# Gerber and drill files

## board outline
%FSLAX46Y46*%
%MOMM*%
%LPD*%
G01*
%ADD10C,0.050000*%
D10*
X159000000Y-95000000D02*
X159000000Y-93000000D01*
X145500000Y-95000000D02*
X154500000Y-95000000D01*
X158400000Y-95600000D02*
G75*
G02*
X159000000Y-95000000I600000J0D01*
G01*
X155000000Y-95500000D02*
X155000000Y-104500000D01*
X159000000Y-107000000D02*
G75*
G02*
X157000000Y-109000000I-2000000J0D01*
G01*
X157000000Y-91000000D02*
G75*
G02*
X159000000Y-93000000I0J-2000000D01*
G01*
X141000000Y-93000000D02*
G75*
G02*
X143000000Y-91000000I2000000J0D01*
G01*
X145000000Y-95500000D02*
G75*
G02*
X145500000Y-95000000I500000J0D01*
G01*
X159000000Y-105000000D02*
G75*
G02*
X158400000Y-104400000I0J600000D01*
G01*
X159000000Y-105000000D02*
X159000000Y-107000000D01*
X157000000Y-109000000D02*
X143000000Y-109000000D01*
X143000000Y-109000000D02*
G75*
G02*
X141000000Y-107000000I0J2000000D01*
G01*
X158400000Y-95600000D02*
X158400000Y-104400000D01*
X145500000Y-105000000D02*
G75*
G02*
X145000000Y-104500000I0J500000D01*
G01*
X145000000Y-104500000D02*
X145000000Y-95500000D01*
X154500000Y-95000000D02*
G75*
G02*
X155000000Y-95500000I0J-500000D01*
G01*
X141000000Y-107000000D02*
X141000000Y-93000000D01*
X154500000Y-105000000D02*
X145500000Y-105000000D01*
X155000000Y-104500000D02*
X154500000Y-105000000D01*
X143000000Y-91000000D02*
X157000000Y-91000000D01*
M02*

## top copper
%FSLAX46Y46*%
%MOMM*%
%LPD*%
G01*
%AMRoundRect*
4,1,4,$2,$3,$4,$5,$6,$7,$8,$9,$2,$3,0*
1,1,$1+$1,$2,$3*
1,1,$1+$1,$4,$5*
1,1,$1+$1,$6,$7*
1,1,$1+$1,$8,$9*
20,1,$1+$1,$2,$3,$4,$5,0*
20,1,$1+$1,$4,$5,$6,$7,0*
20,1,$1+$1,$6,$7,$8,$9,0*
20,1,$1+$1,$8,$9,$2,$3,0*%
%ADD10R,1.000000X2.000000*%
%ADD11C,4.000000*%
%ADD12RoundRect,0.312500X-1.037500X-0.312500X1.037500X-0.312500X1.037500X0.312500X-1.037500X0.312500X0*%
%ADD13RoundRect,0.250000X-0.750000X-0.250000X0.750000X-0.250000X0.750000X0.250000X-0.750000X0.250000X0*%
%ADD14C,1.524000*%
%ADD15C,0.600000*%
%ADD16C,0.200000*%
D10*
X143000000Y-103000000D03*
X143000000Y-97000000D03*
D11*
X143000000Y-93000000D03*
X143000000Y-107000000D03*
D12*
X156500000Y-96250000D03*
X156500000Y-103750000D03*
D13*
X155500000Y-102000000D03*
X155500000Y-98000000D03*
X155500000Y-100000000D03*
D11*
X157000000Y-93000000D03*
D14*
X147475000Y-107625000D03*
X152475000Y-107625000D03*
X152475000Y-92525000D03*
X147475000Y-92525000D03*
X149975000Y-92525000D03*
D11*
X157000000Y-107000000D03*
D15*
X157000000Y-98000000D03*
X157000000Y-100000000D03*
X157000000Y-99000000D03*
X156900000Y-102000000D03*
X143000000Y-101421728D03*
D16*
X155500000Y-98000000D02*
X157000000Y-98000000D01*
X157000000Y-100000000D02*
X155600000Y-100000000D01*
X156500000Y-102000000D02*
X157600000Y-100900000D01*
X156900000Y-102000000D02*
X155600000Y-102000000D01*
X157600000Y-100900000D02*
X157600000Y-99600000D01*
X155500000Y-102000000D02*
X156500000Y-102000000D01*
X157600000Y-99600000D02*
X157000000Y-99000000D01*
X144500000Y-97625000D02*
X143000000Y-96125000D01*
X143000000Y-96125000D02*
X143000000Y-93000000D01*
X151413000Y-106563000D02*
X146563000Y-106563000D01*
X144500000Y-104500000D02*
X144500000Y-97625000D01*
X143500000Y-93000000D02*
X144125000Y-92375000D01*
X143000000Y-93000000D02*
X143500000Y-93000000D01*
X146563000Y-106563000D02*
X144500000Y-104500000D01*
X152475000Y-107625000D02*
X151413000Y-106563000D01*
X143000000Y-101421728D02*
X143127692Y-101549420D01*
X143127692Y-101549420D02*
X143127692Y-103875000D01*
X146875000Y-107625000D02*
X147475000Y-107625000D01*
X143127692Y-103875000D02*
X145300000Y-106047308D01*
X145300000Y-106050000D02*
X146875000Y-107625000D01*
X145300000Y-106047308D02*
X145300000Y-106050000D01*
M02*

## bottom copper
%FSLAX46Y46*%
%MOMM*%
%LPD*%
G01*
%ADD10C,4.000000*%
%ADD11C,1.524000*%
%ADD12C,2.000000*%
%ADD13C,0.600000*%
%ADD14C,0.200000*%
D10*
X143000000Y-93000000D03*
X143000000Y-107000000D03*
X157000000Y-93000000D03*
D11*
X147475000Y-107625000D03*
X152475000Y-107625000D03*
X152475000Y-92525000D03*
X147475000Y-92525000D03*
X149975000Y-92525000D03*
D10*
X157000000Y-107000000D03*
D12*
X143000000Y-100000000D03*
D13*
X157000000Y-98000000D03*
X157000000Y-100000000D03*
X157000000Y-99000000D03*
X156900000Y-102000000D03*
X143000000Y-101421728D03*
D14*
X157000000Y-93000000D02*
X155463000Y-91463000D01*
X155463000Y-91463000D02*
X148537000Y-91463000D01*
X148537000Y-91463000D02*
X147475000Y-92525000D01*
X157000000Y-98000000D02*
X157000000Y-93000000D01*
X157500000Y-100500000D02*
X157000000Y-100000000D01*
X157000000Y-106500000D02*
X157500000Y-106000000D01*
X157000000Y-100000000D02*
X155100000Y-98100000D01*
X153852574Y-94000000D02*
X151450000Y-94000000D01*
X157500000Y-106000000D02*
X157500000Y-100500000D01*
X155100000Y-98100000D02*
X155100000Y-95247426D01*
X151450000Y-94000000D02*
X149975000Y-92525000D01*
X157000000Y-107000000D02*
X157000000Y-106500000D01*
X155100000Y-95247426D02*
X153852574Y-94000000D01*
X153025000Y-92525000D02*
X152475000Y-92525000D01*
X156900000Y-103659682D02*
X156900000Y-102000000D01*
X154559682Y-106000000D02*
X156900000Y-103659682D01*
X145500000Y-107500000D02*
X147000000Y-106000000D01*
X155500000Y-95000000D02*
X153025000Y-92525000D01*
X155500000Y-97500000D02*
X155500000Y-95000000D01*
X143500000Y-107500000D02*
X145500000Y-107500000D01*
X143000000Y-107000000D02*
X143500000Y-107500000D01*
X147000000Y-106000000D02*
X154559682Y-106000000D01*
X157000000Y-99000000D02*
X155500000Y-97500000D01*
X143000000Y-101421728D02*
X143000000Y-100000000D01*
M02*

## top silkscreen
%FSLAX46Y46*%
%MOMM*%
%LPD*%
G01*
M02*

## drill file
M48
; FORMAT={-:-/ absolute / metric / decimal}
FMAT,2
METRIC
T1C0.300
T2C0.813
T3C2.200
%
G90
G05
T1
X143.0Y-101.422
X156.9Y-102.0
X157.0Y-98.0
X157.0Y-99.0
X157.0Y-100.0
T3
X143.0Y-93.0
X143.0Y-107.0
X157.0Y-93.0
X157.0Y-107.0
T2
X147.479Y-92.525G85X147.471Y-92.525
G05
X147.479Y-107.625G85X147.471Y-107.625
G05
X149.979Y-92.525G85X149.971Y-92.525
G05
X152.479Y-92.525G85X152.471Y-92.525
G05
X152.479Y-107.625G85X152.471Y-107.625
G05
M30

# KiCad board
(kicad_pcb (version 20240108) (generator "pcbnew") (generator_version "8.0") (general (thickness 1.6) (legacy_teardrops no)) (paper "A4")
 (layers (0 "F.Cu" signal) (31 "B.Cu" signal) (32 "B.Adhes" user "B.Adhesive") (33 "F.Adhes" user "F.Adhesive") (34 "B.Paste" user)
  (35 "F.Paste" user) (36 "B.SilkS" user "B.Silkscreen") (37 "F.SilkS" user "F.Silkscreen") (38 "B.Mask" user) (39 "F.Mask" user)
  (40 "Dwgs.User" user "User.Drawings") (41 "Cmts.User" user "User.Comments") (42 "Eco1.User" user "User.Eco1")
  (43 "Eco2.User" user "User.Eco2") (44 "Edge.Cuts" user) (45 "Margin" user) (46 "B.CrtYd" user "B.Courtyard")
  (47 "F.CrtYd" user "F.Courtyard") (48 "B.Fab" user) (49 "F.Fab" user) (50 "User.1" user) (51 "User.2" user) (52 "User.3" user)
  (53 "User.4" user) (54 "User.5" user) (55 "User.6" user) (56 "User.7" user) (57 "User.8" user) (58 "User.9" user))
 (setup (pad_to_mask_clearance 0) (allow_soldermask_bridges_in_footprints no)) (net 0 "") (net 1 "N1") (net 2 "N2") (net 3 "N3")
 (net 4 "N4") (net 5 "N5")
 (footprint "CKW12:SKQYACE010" (layer "F.Cu") (at 143 100 -90)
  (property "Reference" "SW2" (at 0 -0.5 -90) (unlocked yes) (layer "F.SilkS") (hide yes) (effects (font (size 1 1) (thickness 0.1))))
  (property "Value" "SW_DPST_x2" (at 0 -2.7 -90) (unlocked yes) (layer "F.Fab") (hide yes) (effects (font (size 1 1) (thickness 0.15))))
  (pad "1" smd rect (at 3 0 270) (size 2 1) (layers "F.Cu" "F.Paste" "F.Mask") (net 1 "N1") (thermal_bridge_angle 45))
  (pad "2" smd rect (at -3 0 270) (size 2 1) (layers "F.Cu" "F.Paste" "F.Mask") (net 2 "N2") (thermal_bridge_angle 45)))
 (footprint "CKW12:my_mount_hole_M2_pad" (layer "F.Cu") (at 143 93)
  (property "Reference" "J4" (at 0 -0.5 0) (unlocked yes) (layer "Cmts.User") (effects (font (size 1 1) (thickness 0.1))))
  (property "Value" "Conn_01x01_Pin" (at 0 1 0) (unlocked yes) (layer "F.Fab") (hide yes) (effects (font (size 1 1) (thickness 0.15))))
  (pad "" thru_hole circle (at 0 0) (size 4 4) (drill 2.2) (layers "*.Cu" "*.Mask") (remove_unused_layers no) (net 2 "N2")))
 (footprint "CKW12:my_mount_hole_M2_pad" (layer "F.Cu") (at 143 107)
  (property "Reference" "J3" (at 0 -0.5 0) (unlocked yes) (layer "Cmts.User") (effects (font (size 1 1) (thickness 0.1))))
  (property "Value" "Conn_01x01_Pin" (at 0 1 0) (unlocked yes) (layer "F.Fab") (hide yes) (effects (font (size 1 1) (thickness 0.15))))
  (pad "" thru_hole circle (at 0 0) (size 4 4) (drill 2.2) (layers "*.Cu" "*.Mask") (remove_unused_layers no) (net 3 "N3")))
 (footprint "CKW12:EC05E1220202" (layer "F.Cu") (at 150 100)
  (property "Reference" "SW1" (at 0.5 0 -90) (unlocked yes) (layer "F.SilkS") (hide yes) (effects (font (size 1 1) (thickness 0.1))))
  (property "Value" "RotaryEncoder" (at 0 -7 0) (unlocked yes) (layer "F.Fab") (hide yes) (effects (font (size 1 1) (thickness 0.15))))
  (pad "" smd roundrect (at 6.5 -3.75) (size 2.7 1.25) (layers "F.Cu" "F.Paste" "F.Mask") (roundrect_rratio 0.25) (thermal_bridge_angle 45))
  (pad "" smd roundrect (at 6.5 3.75) (size 2.7 1.25) (layers "F.Cu" "F.Paste" "F.Mask") (roundrect_rratio 0.25) (thermal_bridge_angle 45))
  (pad "A" smd roundrect (at 5.5 2) (size 2 1) (layers "F.Cu" "F.Paste" "F.Mask") (roundrect_rratio 0.25) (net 3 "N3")
   (thermal_bridge_angle 45))
  (pad "B" smd roundrect (at 5.5 -2) (size 2 1) (layers "F.Cu" "F.Paste" "F.Mask") (roundrect_rratio 0.25) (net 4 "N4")
   (thermal_bridge_angle 45))
  (pad "C" smd roundrect (at 5.5 0) (size 2 1) (layers "F.Cu" "F.Paste" "F.Mask") (roundrect_rratio 0.25) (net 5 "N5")
   (thermal_bridge_angle 45)))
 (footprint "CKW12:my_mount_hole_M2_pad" (layer "F.Cu") (at 157 93)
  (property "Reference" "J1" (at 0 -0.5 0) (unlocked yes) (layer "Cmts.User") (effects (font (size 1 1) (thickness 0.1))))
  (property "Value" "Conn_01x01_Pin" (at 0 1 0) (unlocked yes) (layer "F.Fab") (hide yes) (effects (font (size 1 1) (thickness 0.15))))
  (pad "" thru_hole circle (at 0 0) (size 4 4) (drill 2.2) (layers "*.Cu" "*.Mask") (remove_unused_layers no) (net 4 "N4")))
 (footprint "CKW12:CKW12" (layer "F.Cu") (at 150 100 180)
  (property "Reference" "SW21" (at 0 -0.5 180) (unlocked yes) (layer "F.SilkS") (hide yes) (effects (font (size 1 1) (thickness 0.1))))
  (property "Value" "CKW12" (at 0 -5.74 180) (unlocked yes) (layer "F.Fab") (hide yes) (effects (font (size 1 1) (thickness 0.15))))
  (pad "1" thru_hole circle (at 2.525 -7.625 180) (size 1.524 1.524) (drill oval 0.82 0.8128) (layers "*.Cu" "*.Mask")
   (remove_unused_layers no) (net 1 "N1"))
  (pad "2" thru_hole circle (at -2.475 -7.625 180) (size 1.524 1.524) (drill oval 0.82 0.8128) (layers "*.Cu" "*.Mask")
   (remove_unused_layers no) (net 2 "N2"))
  (pad "A" thru_hole circle (at -2.475 7.475 180) (size 1.524 1.524) (drill oval 0.82 0.8128) (layers "*.Cu" "*.Mask")
   (remove_unused_layers no) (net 3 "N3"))
  (pad "B" thru_hole circle (at 2.525 7.475 180) (size 1.524 1.524) (drill oval 0.82 0.8128) (layers "*.Cu" "*.Mask")
   (remove_unused_layers no) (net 4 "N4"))
  (pad "C" thru_hole circle (at 0.025 7.475 180) (size 1.524 1.524) (drill oval 0.82 0.8128) (layers "*.Cu" "*.Mask")
   (remove_unused_layers no) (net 5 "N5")))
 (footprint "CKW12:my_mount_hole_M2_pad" (layer "F.Cu") (at 157 107)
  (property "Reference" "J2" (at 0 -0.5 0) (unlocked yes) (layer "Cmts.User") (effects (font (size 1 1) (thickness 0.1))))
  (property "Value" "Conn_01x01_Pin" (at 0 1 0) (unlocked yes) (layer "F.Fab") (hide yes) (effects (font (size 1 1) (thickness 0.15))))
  (pad "" thru_hole circle (at 0 0) (size 4 4) (drill 2.2) (layers "*.Cu" "*.Mask") (remove_unused_layers no) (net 5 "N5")))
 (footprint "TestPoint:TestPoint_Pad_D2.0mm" (layer "B.Cu") (at 143 100 180)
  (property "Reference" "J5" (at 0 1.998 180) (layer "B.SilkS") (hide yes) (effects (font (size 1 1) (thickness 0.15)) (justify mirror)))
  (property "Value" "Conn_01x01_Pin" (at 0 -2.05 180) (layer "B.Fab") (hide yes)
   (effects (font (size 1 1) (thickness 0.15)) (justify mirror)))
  (pad "1" smd circle (at 0 0 180) (size 2 2) (layers "B.Cu" "B.Mask") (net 1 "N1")))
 (gr_line (start 159 95) (end 159 93) (stroke (width 0.05) (type default)) (layer "Edge.Cuts"))
 (gr_line (start 145.5 95) (end 154.5 95) (stroke (width 0.05) (type default)) (layer "Edge.Cuts"))
 (gr_arc (start 158.4 95.6) (mid 158.575736 95.175736) (end 159 95) (stroke (width 0.05) (type default)) (layer "Edge.Cuts"))
 (gr_line (start 155 95.5) (end 155 104.5) (stroke (width 0.05) (type default)) (layer "Edge.Cuts"))
 (gr_arc (start 159 107) (mid 158.414214 108.414214) (end 157 109) (stroke (width 0.05) (type default)) (layer "Edge.Cuts"))
 (gr_arc (start 157 91) (mid 158.414214 91.585786) (end 159 93) (stroke (width 0.05) (type default)) (layer "Edge.Cuts"))
 (gr_arc (start 141 93) (mid 141.585786 91.585786) (end 143 91) (stroke (width 0.05) (type default)) (layer "Edge.Cuts"))
 (gr_arc (start 145 95.5) (mid 145.146447 95.146447) (end 145.5 95) (stroke (width 0.05) (type default)) (layer "Edge.Cuts"))
 (gr_arc (start 159 105) (mid 158.575736 104.824264) (end 158.4 104.4) (stroke (width 0.05) (type default)) (layer "Edge.Cuts"))
 (gr_line (start 159 105) (end 159 107) (stroke (width 0.05) (type default)) (layer "Edge.Cuts"))
 (gr_line (start 157 109) (end 143 109) (stroke (width 0.05) (type default)) (layer "Edge.Cuts"))
 (gr_arc (start 143 109) (mid 141.585786 108.414214) (end 141 107) (stroke (width 0.05) (type default)) (layer "Edge.Cuts"))
 (gr_line (start 158.4 95.6) (end 158.4 104.4) (stroke (width 0.05) (type default)) (layer "Edge.Cuts"))
 (gr_arc (start 145.5 105) (mid 145.146447 104.853553) (end 145 104.5) (stroke (width 0.05) (type default)) (layer "Edge.Cuts"))
 (gr_line (start 145 104.5) (end 145 95.5) (stroke (width 0.05) (type default)) (layer "Edge.Cuts"))
 (gr_arc (start 154.5 95) (mid 154.853553 95.146447) (end 155 95.5) (stroke (width 0.05) (type default)) (layer "Edge.Cuts"))
 (gr_line (start 141 107) (end 141 93) (stroke (width 0.05) (type default)) (layer "Edge.Cuts"))
 (gr_line (start 154.5 105) (end 145.5 105) (stroke (width 0.05) (type default)) (layer "Edge.Cuts"))
 (gr_line (start 155 104.5) (end 154.5 105) (stroke (width 0.05) (type default)) (layer "Edge.Cuts"))
 (gr_line (start 143 91) (end 157 91) (stroke (width 0.05) (type default)) (layer "Edge.Cuts"))
 (segment (start 155.5 98) (end 157 98) (width 0.2) (layer "F.Cu") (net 4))
 (via (at 157 98) (size 0.6) (drill 0.3) (layers "F.Cu" "B.Cu") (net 4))
 (segment (start 157 93) (end 155.463 91.463) (width 0.2) (layer "B.Cu") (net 4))
 (segment (start 155.463 91.463) (end 148.537 91.463) (width 0.2) (layer "B.Cu") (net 4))
 (segment (start 148.537 91.463) (end 147.475 92.525) (width 0.2) (layer "B.Cu") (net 4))
 (segment (start 157 98) (end 157 93) (width 0.2) (layer "B.Cu") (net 4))
 (segment (start 157 100) (end 155.6 100) (width 0.2) (layer "F.Cu") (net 5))
 (via (at 157 100) (size 0.6) (drill 0.3) (layers "F.Cu" "B.Cu") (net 5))
 (segment (start 157.5 100.5) (end 157 100) (width 0.2) (layer "B.Cu") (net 5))
 (segment (start 157 106.5) (end 157.5 106) (width 0.2) (layer "B.Cu") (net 5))
 (segment (start 157 100) (end 155.1 98.1) (width 0.2) (layer "B.Cu") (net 5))
 (segment (start 153.852574 94) (end 151.45 94) (width 0.2) (layer "B.Cu") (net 5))
 (segment (start 157.5 106) (end 157.5 100.5) (width 0.2) (layer "B.Cu") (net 5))
 (segment (start 155.1 98.1) (end 155.1 95.247426) (width 0.2) (layer "B.Cu") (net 5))
 (segment (start 151.45 94) (end 149.975 92.525) (width 0.2) (layer "B.Cu") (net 5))
 (segment (start 157 107) (end 157 106.5) (width 0.2) (layer "B.Cu") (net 5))
 (segment (start 155.1 95.247426) (end 153.852574 94) (width 0.2) (layer "B.Cu") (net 5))
 (segment (start 156.5 102) (end 157.6 100.9) (width 0.2) (layer "F.Cu") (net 3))
 (segment (start 156.9 102) (end 155.6 102) (width 0.2) (layer "F.Cu") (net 3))
 (segment (start 157.6 100.9) (end 157.6 99.6) (width 0.2) (layer "F.Cu") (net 3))
 (segment (start 155.5 102) (end 156.5 102) (width 0.2) (layer "F.Cu") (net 3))
 (segment (start 157.6 99.6) (end 157 99) (width 0.2) (layer "F.Cu") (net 3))
 (via (at 157 99) (size 0.6) (drill 0.3) (layers "F.Cu" "B.Cu") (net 3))
 (via (at 156.9 102) (size 0.6) (drill 0.3) (layers "F.Cu" "B.Cu") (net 3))
 (segment (start 153.025 92.525) (end 152.475 92.525) (width 0.2) (layer "B.Cu") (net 3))
 (segment (start 156.9 103.659682) (end 156.9 102) (width 0.2) (layer "B.Cu") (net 3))
 (segment (start 154.559682 106) (end 156.9 103.659682) (width 0.2) (layer "B.Cu") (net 3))
 (segment (start 145.5 107.5) (end 147 106) (width 0.2) (layer "B.Cu") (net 3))
 (segment (start 155.5 95) (end 153.025 92.525) (width 0.2) (layer "B.Cu") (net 3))
 (segment (start 155.5 97.5) (end 155.5 95) (width 0.2) (layer "B.Cu") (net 3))
 (segment (start 143.5 107.5) (end 145.5 107.5) (width 0.2) (layer "B.Cu") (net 3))
 (segment (start 143 107) (end 143.5 107.5) (width 0.2) (layer "B.Cu") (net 3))
 (segment (start 147 106) (end 154.559682 106) (width 0.2) (layer "B.Cu") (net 3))
 (segment (start 157 99) (end 155.5 97.5) (width 0.2) (layer "B.Cu") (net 3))
 (segment (start 144.5 97.625) (end 143 96.125) (width 0.2) (layer "F.Cu") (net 2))
 (segment (start 143 96.125) (end 143 93) (width 0.2) (layer "F.Cu") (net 2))
 (segment (start 151.413 106.563) (end 146.563 106.563) (width 0.2) (layer "F.Cu") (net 2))
 (segment (start 144.5 104.5) (end 144.5 97.625) (width 0.2) (layer "F.Cu") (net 2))
 (segment (start 143.5 93) (end 144.125 92.375) (width 0.2) (layer "F.Cu") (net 2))
 (segment (start 143 93) (end 143.5 93) (width 0.2) (layer "F.Cu") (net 2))
 (segment (start 146.563 106.563) (end 144.5 104.5) (width 0.2) (layer "F.Cu") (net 2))
 (segment (start 152.475 107.625) (end 151.413 106.563) (width 0.2) (layer "F.Cu") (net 2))
 (segment (start 143 101.421728) (end 143.127692 101.54942) (width 0.2) (layer "F.Cu") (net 1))
 (segment (start 143.127692 101.54942) (end 143.127692 103.875) (width 0.2) (layer "F.Cu") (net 1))
 (segment (start 146.875 107.625) (end 147.475 107.625) (width 0.2) (layer "F.Cu") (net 1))
 (segment (start 143.127692 103.875) (end 145.3 106.047308) (width 0.2) (layer "F.Cu") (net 1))
 (segment (start 145.3 106.05) (end 146.875 107.625) (width 0.2) (layer "F.Cu") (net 1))
 (segment (start 145.3 106.047308) (end 145.3 106.05) (width 0.2) (layer "F.Cu") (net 1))
 (via (at 143 101.421728) (size 0.6) (drill 0.3) (layers "F.Cu" "B.Cu") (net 1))
 (segment (start 143 101.421728) (end 143 100) (width 0.2) (layer "B.Cu") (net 1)))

